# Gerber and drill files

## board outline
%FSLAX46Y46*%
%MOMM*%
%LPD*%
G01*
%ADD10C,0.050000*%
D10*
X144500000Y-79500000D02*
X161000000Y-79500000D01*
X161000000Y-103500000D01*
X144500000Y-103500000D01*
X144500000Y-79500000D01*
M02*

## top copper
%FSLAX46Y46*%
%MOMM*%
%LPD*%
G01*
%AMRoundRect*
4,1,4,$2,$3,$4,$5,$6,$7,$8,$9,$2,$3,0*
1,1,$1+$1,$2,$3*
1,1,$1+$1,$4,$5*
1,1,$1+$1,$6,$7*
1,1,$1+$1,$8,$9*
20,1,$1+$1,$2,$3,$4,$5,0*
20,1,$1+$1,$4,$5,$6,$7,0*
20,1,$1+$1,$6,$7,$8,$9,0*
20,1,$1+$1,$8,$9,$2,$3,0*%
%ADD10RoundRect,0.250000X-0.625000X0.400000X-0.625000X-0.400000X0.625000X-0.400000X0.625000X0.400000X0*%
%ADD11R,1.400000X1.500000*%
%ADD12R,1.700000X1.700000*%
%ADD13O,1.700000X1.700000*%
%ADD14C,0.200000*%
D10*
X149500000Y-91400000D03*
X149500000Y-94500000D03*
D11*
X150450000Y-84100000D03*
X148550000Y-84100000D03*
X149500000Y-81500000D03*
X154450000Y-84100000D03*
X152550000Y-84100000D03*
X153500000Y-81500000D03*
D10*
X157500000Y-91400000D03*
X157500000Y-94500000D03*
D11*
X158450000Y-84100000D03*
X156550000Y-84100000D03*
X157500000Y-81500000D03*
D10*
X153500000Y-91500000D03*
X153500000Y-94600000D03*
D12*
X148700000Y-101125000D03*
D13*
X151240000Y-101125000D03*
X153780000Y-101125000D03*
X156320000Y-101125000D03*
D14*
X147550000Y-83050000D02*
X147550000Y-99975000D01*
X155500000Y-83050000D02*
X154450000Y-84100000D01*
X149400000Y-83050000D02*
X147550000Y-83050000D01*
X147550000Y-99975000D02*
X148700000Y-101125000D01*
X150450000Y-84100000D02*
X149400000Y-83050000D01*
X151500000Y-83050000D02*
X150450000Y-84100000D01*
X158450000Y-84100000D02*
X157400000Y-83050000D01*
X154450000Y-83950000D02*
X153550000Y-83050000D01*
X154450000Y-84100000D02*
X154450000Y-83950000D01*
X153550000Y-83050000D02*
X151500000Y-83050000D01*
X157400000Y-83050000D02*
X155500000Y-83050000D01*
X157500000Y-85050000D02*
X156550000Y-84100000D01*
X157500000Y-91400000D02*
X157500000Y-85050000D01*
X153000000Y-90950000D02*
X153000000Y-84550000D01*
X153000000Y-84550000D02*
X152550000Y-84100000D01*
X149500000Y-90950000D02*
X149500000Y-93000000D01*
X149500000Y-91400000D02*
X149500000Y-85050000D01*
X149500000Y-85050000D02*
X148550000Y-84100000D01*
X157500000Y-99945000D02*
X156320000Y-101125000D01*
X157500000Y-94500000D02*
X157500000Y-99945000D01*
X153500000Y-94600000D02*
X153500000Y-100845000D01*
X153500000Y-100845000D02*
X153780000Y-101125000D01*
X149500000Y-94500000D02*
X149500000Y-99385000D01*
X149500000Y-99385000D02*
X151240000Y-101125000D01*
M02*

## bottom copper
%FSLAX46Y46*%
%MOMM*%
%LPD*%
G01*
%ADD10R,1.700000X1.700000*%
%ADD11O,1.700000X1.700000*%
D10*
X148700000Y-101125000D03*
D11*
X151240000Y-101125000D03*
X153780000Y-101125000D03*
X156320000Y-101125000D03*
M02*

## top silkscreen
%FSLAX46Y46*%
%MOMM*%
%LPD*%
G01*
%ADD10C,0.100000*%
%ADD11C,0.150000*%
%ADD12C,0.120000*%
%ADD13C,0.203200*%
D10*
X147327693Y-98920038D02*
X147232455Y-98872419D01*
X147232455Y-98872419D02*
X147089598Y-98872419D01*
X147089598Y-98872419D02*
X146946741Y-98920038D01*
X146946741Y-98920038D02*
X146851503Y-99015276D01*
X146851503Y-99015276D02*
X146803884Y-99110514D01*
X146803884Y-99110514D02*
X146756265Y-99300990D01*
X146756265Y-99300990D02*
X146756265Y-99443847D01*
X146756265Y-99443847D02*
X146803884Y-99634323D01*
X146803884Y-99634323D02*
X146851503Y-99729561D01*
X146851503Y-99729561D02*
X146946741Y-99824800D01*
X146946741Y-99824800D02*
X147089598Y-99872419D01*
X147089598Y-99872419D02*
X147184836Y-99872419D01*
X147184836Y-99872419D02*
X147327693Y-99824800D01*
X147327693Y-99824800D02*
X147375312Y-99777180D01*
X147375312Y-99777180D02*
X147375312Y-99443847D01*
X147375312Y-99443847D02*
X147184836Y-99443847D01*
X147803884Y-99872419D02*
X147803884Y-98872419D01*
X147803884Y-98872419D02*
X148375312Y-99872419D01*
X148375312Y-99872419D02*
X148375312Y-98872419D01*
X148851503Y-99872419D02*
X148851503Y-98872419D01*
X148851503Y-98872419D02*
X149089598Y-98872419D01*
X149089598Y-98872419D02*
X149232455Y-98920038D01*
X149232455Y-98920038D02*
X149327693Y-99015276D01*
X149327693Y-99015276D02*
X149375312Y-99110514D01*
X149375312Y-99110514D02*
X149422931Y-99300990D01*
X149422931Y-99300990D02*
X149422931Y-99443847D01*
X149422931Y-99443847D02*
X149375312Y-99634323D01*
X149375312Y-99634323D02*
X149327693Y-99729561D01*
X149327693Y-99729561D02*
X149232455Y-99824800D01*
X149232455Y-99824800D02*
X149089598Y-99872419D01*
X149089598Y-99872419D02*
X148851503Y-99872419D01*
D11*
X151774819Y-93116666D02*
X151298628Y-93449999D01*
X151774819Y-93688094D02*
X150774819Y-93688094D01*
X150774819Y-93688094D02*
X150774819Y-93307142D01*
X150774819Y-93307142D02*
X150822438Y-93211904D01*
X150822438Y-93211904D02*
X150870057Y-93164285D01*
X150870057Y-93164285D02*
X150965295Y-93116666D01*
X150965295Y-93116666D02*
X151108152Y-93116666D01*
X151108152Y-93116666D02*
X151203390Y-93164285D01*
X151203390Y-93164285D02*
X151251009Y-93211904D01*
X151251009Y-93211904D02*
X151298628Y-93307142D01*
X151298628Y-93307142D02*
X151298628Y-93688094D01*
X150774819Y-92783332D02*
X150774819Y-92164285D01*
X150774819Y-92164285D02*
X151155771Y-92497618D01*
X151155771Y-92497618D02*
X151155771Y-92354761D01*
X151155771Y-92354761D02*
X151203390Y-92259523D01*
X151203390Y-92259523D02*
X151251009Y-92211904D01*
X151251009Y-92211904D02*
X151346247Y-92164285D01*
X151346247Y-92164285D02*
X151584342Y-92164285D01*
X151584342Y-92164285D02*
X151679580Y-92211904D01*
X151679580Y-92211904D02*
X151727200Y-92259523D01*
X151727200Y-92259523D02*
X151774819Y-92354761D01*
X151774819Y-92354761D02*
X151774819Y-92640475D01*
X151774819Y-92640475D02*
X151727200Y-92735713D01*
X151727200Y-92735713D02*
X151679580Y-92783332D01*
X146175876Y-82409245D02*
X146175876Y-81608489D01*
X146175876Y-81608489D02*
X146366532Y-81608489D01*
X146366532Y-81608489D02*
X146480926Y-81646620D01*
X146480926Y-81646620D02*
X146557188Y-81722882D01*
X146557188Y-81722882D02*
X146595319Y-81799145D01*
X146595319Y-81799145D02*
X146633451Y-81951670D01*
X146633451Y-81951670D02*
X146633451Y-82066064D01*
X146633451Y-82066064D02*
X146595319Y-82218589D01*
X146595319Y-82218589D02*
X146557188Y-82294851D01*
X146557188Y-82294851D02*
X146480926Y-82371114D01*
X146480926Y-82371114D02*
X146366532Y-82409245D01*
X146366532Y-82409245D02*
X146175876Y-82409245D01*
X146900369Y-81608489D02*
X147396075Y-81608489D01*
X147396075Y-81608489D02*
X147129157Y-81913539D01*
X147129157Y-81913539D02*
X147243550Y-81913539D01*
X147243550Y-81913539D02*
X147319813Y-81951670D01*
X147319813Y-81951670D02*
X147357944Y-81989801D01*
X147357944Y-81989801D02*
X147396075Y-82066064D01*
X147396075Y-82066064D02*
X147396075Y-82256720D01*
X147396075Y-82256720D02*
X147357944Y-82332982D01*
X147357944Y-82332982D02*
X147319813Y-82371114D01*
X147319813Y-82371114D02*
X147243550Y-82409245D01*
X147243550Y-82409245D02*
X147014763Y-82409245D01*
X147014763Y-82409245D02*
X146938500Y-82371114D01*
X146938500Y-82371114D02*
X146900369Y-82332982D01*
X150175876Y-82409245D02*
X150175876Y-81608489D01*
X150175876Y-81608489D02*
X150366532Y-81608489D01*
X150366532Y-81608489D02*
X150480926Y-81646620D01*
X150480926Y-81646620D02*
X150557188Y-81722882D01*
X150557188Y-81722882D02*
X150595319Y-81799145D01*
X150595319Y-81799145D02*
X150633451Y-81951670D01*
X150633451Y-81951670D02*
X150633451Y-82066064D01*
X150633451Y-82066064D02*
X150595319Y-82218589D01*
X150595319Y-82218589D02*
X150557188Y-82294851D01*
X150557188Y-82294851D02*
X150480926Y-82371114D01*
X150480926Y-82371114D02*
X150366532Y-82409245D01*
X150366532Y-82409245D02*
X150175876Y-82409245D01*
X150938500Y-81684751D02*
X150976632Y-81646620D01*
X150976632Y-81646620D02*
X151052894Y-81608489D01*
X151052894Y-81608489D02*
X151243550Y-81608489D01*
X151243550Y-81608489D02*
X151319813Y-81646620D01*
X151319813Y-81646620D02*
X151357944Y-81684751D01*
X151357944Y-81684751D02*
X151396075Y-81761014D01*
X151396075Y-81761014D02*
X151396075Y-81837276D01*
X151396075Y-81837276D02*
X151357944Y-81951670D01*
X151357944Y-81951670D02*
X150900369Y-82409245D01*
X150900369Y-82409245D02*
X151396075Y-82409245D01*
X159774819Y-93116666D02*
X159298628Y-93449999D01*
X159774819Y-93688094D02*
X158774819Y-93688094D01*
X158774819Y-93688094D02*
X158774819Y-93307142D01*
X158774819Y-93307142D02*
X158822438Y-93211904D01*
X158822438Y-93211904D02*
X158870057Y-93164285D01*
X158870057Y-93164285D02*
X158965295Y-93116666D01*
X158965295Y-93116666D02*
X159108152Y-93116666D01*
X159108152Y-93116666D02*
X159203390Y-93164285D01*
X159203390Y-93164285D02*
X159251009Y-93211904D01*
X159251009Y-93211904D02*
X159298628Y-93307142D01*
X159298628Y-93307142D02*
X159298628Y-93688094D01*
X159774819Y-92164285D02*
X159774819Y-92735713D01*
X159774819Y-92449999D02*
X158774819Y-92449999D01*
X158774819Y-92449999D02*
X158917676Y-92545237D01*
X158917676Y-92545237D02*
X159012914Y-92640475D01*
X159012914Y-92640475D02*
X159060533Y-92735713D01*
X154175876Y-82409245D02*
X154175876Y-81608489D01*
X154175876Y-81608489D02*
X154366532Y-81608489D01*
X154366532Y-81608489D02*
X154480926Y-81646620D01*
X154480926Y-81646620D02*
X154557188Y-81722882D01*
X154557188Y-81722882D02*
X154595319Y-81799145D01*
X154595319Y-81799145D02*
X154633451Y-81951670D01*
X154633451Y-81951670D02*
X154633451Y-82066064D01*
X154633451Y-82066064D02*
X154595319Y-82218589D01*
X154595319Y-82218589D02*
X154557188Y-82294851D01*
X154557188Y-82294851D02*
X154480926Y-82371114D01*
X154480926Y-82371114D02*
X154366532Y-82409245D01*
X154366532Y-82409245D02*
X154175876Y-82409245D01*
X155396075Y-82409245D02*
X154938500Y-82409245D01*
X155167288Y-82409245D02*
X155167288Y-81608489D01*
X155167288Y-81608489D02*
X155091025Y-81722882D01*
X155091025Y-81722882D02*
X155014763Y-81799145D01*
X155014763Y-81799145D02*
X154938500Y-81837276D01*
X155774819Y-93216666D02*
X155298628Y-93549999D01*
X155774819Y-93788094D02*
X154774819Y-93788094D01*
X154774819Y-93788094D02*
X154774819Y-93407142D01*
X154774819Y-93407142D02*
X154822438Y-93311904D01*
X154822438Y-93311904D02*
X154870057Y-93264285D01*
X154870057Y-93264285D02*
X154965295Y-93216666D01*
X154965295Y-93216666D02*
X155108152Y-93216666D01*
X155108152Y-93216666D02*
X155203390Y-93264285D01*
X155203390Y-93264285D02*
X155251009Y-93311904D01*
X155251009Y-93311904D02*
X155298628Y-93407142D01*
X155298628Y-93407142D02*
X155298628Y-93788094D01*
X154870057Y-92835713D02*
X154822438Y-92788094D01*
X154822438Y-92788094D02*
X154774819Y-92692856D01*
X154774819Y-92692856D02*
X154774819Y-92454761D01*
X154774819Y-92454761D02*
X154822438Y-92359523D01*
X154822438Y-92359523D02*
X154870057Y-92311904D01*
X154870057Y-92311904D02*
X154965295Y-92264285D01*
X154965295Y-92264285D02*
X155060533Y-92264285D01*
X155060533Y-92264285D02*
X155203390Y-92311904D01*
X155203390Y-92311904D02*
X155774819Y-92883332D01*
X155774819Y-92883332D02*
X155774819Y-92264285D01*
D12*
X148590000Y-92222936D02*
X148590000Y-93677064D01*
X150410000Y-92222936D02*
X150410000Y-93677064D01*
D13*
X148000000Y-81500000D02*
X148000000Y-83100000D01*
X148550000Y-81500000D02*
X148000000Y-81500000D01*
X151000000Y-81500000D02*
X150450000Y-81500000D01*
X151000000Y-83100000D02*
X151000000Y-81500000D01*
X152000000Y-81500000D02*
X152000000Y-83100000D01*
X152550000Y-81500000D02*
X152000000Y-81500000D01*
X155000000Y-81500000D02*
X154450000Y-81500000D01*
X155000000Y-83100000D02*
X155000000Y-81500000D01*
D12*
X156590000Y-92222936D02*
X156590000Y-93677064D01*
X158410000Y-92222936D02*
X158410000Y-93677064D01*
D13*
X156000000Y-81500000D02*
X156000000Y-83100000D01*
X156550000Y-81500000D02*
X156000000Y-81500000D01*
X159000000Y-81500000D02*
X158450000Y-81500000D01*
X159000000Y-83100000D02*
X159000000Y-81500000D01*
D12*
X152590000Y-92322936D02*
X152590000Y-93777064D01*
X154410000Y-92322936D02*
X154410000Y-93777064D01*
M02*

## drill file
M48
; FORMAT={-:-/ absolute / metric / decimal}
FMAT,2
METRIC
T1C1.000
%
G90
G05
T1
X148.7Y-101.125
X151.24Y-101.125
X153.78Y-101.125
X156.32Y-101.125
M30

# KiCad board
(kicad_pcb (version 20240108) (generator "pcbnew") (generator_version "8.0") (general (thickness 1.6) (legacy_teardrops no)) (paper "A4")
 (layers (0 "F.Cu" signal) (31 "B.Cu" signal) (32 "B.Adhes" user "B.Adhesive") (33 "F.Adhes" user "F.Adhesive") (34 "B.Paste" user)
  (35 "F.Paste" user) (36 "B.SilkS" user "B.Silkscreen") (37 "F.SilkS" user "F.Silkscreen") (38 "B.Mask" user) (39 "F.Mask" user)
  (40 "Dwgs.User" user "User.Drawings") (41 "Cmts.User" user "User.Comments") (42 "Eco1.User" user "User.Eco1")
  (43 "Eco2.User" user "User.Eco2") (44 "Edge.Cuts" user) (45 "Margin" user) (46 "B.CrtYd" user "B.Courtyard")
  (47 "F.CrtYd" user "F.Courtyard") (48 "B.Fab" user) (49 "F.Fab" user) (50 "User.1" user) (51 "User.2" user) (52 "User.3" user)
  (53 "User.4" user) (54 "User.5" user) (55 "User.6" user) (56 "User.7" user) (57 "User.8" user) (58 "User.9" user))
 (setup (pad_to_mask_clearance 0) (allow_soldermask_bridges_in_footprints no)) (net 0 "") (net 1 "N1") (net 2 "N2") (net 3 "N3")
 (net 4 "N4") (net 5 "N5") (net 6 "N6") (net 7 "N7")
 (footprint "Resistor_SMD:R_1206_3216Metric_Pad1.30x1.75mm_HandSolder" (layer "F.Cu") (at 149.5 92.95 -90)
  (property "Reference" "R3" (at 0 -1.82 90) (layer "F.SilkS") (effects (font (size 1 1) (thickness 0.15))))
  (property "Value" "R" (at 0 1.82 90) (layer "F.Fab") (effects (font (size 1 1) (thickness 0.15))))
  (fp_line (start -0.727064 0.91) (end 0.727064 0.91) (stroke (width 0.12) (type solid)) (layer "F.SilkS"))
  (fp_line (start -0.727064 -0.91) (end 0.727064 -0.91) (stroke (width 0.12) (type solid)) (layer "F.SilkS"))
  (pad "1" smd roundrect (at -1.55 0 270) (size 1.3 1.75) (layers "F.Cu" "F.Paste" "F.Mask") (roundrect_rratio 0.192308) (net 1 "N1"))
  (pad "2" smd roundrect (at 1.55 0 270) (size 1.3 1.75) (layers "F.Cu" "F.Paste" "F.Mask") (roundrect_rratio 0.192308) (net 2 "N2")))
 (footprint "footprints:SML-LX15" (layer "F.Cu") (at 149.5 83)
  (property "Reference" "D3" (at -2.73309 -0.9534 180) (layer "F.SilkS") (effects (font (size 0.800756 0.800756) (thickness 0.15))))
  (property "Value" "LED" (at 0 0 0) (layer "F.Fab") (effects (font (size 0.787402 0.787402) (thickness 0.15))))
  (fp_line (start -1.5 -1.5) (end -1.5 0.1) (stroke (width 0.2032) (type solid)) (layer "F.SilkS"))
  (fp_line (start -0.95 -1.5) (end -1.5 -1.5) (stroke (width 0.2032) (type solid)) (layer "F.SilkS"))
  (fp_line (start 1.5 -1.5) (end 0.95 -1.5) (stroke (width 0.2032) (type solid)) (layer "F.SilkS"))
  (fp_line (start 1.5 0.1) (end 1.5 -1.5) (stroke (width 0.2032) (type solid)) (layer "F.SilkS"))
  (pad "1" smd rect (at 0.95 1.1) (size 1.4 1.5) (layers "F.Cu" "F.Paste" "F.Mask") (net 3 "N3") (solder_mask_margin 0.102))
  (pad "2" smd rect (at -0.95 1.1) (size 1.4 1.5) (layers "F.Cu" "F.Paste" "F.Mask") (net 1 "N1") (solder_mask_margin 0.102))
  (pad "3" smd rect (at 0 -1.5) (size 1.4 1.5) (layers "F.Cu" "F.Paste" "F.Mask") (solder_mask_margin 0.102)))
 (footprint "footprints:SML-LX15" (layer "F.Cu") (at 153.5 83)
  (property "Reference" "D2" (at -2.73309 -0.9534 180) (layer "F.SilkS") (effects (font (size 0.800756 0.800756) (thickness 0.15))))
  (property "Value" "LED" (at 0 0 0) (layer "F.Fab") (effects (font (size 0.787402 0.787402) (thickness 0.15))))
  (fp_line (start -1.5 -1.5) (end -1.5 0.1) (stroke (width 0.2032) (type solid)) (layer "F.SilkS"))
  (fp_line (start -0.95 -1.5) (end -1.5 -1.5) (stroke (width 0.2032) (type solid)) (layer "F.SilkS"))
  (fp_line (start 1.5 -1.5) (end 0.95 -1.5) (stroke (width 0.2032) (type solid)) (layer "F.SilkS"))
  (fp_line (start 1.5 0.1) (end 1.5 -1.5) (stroke (width 0.2032) (type solid)) (layer "F.SilkS"))
  (pad "1" smd rect (at 0.95 1.1) (size 1.4 1.5) (layers "F.Cu" "F.Paste" "F.Mask") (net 3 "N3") (solder_mask_margin 0.102))
  (pad "2" smd rect (at -0.95 1.1) (size 1.4 1.5) (layers "F.Cu" "F.Paste" "F.Mask") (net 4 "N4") (solder_mask_margin 0.102))
  (pad "3" smd rect (at 0 -1.5) (size 1.4 1.5) (layers "F.Cu" "F.Paste" "F.Mask") (solder_mask_margin 0.102)))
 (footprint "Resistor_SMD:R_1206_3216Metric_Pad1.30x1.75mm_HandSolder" (layer "F.Cu") (at 157.5 92.95 -90)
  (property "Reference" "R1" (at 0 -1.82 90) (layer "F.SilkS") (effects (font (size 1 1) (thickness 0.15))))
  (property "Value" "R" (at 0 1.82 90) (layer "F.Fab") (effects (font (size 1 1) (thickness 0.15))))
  (fp_line (start -0.727064 0.91) (end 0.727064 0.91) (stroke (width 0.12) (type solid)) (layer "F.SilkS"))
  (fp_line (start -0.727064 -0.91) (end 0.727064 -0.91) (stroke (width 0.12) (type solid)) (layer "F.SilkS"))
  (pad "1" smd roundrect (at -1.55 0 270) (size 1.3 1.75) (layers "F.Cu" "F.Paste" "F.Mask") (roundrect_rratio 0.192308) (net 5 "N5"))
  (pad "2" smd roundrect (at 1.55 0 270) (size 1.3 1.75) (layers "F.Cu" "F.Paste" "F.Mask") (roundrect_rratio 0.192308) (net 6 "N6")))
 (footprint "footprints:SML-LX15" (layer "F.Cu") (at 157.5 83)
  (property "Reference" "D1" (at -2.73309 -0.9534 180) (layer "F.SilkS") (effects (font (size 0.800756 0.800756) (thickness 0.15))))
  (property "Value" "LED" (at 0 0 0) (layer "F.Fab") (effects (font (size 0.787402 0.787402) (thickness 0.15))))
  (fp_line (start -1.5 -1.5) (end -1.5 0.1) (stroke (width 0.2032) (type solid)) (layer "F.SilkS"))
  (fp_line (start -0.95 -1.5) (end -1.5 -1.5) (stroke (width 0.2032) (type solid)) (layer "F.SilkS"))
  (fp_line (start 1.5 -1.5) (end 0.95 -1.5) (stroke (width 0.2032) (type solid)) (layer "F.SilkS"))
  (fp_line (start 1.5 0.1) (end 1.5 -1.5) (stroke (width 0.2032) (type solid)) (layer "F.SilkS"))
  (pad "1" smd rect (at 0.95 1.1) (size 1.4 1.5) (layers "F.Cu" "F.Paste" "F.Mask") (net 3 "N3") (solder_mask_margin 0.102))
  (pad "2" smd rect (at -0.95 1.1) (size 1.4 1.5) (layers "F.Cu" "F.Paste" "F.Mask") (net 5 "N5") (solder_mask_margin 0.102))
  (pad "3" smd rect (at 0 -1.5) (size 1.4 1.5) (layers "F.Cu" "F.Paste" "F.Mask") (solder_mask_margin 0.102)))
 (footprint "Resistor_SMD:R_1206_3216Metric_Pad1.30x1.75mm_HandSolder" (layer "F.Cu") (at 153.5 93.05 -90)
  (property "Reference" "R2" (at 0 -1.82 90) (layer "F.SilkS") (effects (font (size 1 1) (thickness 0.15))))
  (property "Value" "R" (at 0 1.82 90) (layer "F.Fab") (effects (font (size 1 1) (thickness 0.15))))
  (fp_line (start -0.727064 0.91) (end 0.727064 0.91) (stroke (width 0.12) (type solid)) (layer "F.SilkS"))
  (fp_line (start -0.727064 -0.91) (end 0.727064 -0.91) (stroke (width 0.12) (type solid)) (layer "F.SilkS"))
  (pad "1" smd roundrect (at -1.55 0 270) (size 1.3 1.75) (layers "F.Cu" "F.Paste" "F.Mask") (roundrect_rratio 0.192308) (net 4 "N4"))
  (pad "2" smd roundrect (at 1.55 0 270) (size 1.3 1.75) (layers "F.Cu" "F.Paste" "F.Mask") (roundrect_rratio 0.192308) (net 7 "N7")))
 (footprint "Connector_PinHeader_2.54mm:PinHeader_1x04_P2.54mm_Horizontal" (layer "B.Cu") (at 148.7 101.125 -90)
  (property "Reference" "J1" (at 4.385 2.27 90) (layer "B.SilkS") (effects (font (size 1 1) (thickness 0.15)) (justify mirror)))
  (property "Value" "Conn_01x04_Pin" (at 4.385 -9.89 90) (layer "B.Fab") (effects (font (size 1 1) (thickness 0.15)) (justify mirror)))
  (pad "1" thru_hole rect (at 0 0 270) (size 1.7 1.7) (drill 1) (layers "*.Cu" "*.Mask") (remove_unused_layers no) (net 3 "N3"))
  (pad "2" thru_hole oval (at 0 -2.54 270) (size 1.7 1.7) (drill 1) (layers "*.Cu" "*.Mask") (remove_unused_layers no) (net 2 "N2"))
  (pad "3" thru_hole oval (at 0 -5.08 270) (size 1.7 1.7) (drill 1) (layers "*.Cu" "*.Mask") (remove_unused_layers no) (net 7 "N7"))
  (pad "4" thru_hole oval (at 0 -7.62 270) (size 1.7 1.7) (drill 1) (layers "*.Cu" "*.Mask") (remove_unused_layers no) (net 6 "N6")))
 (gr_rect (start 144.5 79.5) (end 161 103.5) (stroke (width 0.05) (type default)) (fill none) (layer "Edge.Cuts"))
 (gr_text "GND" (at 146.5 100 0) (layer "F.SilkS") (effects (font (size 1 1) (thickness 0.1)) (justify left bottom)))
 (segment (start 147.55 83.05) (end 147.55 99.975) (width 0.2) (layer "F.Cu") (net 3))
 (segment (start 155.5 83.05) (end 154.45 84.1) (width 0.2) (layer "F.Cu") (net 3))
 (segment (start 149.4 83.05) (end 147.55 83.05) (width 0.2) (layer "F.Cu") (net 3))
 (segment (start 147.55 99.975) (end 148.7 101.125) (width 0.2) (layer "F.Cu") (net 3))
 (segment (start 150.45 84.1) (end 149.4 83.05) (width 0.2) (layer "F.Cu") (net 3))
 (segment (start 151.5 83.05) (end 150.45 84.1) (width 0.2) (layer "F.Cu") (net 3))
 (segment (start 158.45 84.1) (end 157.4 83.05) (width 0.2) (layer "F.Cu") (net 3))
 (segment (start 154.45 83.95) (end 153.55 83.05) (width 0.2) (layer "F.Cu") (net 3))
 (segment (start 154.45 84.1) (end 154.45 83.95) (width 0.2) (layer "F.Cu") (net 3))
 (segment (start 153.55 83.05) (end 151.5 83.05) (width 0.2) (layer "F.Cu") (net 3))
 (segment (start 157.4 83.05) (end 155.5 83.05) (width 0.2) (layer "F.Cu") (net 3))
 (segment (start 157.5 85.05) (end 156.55 84.1) (width 0.2) (layer "F.Cu") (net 5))
 (segment (start 157.5 91.4) (end 157.5 85.05) (width 0.2) (layer "F.Cu") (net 5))
 (segment (start 153 90.95) (end 153 84.55) (width 0.2) (layer "F.Cu") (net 4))
 (segment (start 153 84.55) (end 152.55 84.1) (width 0.2) (layer "F.Cu") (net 4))
 (segment (start 149.5 90.95) (end 149.5 93) (width 0.2) (layer "F.Cu") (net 1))
 (segment (start 149.5 91.4) (end 149.5 85.05) (width 0.2) (layer "F.Cu") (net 1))
 (segment (start 149.5 85.05) (end 148.55 84.1) (width 0.2) (layer "F.Cu") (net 1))
 (segment (start 157.5 99.945) (end 156.32 101.125) (width 0.2) (layer "F.Cu") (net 6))
 (segment (start 157.5 94.5) (end 157.5 99.945) (width 0.2) (layer "F.Cu") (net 6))
 (segment (start 153.5 94.6) (end 153.5 100.845) (width 0.2) (layer "F.Cu") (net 7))
 (segment (start 153.5 100.845) (end 153.78 101.125) (width 0.2) (layer "F.Cu") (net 7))
 (segment (start 149.5 94.5) (end 149.5 99.385) (width 0.2) (layer "F.Cu") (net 2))
 (segment (start 149.5 99.385) (end 151.24 101.125) (width 0.2) (layer "F.Cu") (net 2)))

